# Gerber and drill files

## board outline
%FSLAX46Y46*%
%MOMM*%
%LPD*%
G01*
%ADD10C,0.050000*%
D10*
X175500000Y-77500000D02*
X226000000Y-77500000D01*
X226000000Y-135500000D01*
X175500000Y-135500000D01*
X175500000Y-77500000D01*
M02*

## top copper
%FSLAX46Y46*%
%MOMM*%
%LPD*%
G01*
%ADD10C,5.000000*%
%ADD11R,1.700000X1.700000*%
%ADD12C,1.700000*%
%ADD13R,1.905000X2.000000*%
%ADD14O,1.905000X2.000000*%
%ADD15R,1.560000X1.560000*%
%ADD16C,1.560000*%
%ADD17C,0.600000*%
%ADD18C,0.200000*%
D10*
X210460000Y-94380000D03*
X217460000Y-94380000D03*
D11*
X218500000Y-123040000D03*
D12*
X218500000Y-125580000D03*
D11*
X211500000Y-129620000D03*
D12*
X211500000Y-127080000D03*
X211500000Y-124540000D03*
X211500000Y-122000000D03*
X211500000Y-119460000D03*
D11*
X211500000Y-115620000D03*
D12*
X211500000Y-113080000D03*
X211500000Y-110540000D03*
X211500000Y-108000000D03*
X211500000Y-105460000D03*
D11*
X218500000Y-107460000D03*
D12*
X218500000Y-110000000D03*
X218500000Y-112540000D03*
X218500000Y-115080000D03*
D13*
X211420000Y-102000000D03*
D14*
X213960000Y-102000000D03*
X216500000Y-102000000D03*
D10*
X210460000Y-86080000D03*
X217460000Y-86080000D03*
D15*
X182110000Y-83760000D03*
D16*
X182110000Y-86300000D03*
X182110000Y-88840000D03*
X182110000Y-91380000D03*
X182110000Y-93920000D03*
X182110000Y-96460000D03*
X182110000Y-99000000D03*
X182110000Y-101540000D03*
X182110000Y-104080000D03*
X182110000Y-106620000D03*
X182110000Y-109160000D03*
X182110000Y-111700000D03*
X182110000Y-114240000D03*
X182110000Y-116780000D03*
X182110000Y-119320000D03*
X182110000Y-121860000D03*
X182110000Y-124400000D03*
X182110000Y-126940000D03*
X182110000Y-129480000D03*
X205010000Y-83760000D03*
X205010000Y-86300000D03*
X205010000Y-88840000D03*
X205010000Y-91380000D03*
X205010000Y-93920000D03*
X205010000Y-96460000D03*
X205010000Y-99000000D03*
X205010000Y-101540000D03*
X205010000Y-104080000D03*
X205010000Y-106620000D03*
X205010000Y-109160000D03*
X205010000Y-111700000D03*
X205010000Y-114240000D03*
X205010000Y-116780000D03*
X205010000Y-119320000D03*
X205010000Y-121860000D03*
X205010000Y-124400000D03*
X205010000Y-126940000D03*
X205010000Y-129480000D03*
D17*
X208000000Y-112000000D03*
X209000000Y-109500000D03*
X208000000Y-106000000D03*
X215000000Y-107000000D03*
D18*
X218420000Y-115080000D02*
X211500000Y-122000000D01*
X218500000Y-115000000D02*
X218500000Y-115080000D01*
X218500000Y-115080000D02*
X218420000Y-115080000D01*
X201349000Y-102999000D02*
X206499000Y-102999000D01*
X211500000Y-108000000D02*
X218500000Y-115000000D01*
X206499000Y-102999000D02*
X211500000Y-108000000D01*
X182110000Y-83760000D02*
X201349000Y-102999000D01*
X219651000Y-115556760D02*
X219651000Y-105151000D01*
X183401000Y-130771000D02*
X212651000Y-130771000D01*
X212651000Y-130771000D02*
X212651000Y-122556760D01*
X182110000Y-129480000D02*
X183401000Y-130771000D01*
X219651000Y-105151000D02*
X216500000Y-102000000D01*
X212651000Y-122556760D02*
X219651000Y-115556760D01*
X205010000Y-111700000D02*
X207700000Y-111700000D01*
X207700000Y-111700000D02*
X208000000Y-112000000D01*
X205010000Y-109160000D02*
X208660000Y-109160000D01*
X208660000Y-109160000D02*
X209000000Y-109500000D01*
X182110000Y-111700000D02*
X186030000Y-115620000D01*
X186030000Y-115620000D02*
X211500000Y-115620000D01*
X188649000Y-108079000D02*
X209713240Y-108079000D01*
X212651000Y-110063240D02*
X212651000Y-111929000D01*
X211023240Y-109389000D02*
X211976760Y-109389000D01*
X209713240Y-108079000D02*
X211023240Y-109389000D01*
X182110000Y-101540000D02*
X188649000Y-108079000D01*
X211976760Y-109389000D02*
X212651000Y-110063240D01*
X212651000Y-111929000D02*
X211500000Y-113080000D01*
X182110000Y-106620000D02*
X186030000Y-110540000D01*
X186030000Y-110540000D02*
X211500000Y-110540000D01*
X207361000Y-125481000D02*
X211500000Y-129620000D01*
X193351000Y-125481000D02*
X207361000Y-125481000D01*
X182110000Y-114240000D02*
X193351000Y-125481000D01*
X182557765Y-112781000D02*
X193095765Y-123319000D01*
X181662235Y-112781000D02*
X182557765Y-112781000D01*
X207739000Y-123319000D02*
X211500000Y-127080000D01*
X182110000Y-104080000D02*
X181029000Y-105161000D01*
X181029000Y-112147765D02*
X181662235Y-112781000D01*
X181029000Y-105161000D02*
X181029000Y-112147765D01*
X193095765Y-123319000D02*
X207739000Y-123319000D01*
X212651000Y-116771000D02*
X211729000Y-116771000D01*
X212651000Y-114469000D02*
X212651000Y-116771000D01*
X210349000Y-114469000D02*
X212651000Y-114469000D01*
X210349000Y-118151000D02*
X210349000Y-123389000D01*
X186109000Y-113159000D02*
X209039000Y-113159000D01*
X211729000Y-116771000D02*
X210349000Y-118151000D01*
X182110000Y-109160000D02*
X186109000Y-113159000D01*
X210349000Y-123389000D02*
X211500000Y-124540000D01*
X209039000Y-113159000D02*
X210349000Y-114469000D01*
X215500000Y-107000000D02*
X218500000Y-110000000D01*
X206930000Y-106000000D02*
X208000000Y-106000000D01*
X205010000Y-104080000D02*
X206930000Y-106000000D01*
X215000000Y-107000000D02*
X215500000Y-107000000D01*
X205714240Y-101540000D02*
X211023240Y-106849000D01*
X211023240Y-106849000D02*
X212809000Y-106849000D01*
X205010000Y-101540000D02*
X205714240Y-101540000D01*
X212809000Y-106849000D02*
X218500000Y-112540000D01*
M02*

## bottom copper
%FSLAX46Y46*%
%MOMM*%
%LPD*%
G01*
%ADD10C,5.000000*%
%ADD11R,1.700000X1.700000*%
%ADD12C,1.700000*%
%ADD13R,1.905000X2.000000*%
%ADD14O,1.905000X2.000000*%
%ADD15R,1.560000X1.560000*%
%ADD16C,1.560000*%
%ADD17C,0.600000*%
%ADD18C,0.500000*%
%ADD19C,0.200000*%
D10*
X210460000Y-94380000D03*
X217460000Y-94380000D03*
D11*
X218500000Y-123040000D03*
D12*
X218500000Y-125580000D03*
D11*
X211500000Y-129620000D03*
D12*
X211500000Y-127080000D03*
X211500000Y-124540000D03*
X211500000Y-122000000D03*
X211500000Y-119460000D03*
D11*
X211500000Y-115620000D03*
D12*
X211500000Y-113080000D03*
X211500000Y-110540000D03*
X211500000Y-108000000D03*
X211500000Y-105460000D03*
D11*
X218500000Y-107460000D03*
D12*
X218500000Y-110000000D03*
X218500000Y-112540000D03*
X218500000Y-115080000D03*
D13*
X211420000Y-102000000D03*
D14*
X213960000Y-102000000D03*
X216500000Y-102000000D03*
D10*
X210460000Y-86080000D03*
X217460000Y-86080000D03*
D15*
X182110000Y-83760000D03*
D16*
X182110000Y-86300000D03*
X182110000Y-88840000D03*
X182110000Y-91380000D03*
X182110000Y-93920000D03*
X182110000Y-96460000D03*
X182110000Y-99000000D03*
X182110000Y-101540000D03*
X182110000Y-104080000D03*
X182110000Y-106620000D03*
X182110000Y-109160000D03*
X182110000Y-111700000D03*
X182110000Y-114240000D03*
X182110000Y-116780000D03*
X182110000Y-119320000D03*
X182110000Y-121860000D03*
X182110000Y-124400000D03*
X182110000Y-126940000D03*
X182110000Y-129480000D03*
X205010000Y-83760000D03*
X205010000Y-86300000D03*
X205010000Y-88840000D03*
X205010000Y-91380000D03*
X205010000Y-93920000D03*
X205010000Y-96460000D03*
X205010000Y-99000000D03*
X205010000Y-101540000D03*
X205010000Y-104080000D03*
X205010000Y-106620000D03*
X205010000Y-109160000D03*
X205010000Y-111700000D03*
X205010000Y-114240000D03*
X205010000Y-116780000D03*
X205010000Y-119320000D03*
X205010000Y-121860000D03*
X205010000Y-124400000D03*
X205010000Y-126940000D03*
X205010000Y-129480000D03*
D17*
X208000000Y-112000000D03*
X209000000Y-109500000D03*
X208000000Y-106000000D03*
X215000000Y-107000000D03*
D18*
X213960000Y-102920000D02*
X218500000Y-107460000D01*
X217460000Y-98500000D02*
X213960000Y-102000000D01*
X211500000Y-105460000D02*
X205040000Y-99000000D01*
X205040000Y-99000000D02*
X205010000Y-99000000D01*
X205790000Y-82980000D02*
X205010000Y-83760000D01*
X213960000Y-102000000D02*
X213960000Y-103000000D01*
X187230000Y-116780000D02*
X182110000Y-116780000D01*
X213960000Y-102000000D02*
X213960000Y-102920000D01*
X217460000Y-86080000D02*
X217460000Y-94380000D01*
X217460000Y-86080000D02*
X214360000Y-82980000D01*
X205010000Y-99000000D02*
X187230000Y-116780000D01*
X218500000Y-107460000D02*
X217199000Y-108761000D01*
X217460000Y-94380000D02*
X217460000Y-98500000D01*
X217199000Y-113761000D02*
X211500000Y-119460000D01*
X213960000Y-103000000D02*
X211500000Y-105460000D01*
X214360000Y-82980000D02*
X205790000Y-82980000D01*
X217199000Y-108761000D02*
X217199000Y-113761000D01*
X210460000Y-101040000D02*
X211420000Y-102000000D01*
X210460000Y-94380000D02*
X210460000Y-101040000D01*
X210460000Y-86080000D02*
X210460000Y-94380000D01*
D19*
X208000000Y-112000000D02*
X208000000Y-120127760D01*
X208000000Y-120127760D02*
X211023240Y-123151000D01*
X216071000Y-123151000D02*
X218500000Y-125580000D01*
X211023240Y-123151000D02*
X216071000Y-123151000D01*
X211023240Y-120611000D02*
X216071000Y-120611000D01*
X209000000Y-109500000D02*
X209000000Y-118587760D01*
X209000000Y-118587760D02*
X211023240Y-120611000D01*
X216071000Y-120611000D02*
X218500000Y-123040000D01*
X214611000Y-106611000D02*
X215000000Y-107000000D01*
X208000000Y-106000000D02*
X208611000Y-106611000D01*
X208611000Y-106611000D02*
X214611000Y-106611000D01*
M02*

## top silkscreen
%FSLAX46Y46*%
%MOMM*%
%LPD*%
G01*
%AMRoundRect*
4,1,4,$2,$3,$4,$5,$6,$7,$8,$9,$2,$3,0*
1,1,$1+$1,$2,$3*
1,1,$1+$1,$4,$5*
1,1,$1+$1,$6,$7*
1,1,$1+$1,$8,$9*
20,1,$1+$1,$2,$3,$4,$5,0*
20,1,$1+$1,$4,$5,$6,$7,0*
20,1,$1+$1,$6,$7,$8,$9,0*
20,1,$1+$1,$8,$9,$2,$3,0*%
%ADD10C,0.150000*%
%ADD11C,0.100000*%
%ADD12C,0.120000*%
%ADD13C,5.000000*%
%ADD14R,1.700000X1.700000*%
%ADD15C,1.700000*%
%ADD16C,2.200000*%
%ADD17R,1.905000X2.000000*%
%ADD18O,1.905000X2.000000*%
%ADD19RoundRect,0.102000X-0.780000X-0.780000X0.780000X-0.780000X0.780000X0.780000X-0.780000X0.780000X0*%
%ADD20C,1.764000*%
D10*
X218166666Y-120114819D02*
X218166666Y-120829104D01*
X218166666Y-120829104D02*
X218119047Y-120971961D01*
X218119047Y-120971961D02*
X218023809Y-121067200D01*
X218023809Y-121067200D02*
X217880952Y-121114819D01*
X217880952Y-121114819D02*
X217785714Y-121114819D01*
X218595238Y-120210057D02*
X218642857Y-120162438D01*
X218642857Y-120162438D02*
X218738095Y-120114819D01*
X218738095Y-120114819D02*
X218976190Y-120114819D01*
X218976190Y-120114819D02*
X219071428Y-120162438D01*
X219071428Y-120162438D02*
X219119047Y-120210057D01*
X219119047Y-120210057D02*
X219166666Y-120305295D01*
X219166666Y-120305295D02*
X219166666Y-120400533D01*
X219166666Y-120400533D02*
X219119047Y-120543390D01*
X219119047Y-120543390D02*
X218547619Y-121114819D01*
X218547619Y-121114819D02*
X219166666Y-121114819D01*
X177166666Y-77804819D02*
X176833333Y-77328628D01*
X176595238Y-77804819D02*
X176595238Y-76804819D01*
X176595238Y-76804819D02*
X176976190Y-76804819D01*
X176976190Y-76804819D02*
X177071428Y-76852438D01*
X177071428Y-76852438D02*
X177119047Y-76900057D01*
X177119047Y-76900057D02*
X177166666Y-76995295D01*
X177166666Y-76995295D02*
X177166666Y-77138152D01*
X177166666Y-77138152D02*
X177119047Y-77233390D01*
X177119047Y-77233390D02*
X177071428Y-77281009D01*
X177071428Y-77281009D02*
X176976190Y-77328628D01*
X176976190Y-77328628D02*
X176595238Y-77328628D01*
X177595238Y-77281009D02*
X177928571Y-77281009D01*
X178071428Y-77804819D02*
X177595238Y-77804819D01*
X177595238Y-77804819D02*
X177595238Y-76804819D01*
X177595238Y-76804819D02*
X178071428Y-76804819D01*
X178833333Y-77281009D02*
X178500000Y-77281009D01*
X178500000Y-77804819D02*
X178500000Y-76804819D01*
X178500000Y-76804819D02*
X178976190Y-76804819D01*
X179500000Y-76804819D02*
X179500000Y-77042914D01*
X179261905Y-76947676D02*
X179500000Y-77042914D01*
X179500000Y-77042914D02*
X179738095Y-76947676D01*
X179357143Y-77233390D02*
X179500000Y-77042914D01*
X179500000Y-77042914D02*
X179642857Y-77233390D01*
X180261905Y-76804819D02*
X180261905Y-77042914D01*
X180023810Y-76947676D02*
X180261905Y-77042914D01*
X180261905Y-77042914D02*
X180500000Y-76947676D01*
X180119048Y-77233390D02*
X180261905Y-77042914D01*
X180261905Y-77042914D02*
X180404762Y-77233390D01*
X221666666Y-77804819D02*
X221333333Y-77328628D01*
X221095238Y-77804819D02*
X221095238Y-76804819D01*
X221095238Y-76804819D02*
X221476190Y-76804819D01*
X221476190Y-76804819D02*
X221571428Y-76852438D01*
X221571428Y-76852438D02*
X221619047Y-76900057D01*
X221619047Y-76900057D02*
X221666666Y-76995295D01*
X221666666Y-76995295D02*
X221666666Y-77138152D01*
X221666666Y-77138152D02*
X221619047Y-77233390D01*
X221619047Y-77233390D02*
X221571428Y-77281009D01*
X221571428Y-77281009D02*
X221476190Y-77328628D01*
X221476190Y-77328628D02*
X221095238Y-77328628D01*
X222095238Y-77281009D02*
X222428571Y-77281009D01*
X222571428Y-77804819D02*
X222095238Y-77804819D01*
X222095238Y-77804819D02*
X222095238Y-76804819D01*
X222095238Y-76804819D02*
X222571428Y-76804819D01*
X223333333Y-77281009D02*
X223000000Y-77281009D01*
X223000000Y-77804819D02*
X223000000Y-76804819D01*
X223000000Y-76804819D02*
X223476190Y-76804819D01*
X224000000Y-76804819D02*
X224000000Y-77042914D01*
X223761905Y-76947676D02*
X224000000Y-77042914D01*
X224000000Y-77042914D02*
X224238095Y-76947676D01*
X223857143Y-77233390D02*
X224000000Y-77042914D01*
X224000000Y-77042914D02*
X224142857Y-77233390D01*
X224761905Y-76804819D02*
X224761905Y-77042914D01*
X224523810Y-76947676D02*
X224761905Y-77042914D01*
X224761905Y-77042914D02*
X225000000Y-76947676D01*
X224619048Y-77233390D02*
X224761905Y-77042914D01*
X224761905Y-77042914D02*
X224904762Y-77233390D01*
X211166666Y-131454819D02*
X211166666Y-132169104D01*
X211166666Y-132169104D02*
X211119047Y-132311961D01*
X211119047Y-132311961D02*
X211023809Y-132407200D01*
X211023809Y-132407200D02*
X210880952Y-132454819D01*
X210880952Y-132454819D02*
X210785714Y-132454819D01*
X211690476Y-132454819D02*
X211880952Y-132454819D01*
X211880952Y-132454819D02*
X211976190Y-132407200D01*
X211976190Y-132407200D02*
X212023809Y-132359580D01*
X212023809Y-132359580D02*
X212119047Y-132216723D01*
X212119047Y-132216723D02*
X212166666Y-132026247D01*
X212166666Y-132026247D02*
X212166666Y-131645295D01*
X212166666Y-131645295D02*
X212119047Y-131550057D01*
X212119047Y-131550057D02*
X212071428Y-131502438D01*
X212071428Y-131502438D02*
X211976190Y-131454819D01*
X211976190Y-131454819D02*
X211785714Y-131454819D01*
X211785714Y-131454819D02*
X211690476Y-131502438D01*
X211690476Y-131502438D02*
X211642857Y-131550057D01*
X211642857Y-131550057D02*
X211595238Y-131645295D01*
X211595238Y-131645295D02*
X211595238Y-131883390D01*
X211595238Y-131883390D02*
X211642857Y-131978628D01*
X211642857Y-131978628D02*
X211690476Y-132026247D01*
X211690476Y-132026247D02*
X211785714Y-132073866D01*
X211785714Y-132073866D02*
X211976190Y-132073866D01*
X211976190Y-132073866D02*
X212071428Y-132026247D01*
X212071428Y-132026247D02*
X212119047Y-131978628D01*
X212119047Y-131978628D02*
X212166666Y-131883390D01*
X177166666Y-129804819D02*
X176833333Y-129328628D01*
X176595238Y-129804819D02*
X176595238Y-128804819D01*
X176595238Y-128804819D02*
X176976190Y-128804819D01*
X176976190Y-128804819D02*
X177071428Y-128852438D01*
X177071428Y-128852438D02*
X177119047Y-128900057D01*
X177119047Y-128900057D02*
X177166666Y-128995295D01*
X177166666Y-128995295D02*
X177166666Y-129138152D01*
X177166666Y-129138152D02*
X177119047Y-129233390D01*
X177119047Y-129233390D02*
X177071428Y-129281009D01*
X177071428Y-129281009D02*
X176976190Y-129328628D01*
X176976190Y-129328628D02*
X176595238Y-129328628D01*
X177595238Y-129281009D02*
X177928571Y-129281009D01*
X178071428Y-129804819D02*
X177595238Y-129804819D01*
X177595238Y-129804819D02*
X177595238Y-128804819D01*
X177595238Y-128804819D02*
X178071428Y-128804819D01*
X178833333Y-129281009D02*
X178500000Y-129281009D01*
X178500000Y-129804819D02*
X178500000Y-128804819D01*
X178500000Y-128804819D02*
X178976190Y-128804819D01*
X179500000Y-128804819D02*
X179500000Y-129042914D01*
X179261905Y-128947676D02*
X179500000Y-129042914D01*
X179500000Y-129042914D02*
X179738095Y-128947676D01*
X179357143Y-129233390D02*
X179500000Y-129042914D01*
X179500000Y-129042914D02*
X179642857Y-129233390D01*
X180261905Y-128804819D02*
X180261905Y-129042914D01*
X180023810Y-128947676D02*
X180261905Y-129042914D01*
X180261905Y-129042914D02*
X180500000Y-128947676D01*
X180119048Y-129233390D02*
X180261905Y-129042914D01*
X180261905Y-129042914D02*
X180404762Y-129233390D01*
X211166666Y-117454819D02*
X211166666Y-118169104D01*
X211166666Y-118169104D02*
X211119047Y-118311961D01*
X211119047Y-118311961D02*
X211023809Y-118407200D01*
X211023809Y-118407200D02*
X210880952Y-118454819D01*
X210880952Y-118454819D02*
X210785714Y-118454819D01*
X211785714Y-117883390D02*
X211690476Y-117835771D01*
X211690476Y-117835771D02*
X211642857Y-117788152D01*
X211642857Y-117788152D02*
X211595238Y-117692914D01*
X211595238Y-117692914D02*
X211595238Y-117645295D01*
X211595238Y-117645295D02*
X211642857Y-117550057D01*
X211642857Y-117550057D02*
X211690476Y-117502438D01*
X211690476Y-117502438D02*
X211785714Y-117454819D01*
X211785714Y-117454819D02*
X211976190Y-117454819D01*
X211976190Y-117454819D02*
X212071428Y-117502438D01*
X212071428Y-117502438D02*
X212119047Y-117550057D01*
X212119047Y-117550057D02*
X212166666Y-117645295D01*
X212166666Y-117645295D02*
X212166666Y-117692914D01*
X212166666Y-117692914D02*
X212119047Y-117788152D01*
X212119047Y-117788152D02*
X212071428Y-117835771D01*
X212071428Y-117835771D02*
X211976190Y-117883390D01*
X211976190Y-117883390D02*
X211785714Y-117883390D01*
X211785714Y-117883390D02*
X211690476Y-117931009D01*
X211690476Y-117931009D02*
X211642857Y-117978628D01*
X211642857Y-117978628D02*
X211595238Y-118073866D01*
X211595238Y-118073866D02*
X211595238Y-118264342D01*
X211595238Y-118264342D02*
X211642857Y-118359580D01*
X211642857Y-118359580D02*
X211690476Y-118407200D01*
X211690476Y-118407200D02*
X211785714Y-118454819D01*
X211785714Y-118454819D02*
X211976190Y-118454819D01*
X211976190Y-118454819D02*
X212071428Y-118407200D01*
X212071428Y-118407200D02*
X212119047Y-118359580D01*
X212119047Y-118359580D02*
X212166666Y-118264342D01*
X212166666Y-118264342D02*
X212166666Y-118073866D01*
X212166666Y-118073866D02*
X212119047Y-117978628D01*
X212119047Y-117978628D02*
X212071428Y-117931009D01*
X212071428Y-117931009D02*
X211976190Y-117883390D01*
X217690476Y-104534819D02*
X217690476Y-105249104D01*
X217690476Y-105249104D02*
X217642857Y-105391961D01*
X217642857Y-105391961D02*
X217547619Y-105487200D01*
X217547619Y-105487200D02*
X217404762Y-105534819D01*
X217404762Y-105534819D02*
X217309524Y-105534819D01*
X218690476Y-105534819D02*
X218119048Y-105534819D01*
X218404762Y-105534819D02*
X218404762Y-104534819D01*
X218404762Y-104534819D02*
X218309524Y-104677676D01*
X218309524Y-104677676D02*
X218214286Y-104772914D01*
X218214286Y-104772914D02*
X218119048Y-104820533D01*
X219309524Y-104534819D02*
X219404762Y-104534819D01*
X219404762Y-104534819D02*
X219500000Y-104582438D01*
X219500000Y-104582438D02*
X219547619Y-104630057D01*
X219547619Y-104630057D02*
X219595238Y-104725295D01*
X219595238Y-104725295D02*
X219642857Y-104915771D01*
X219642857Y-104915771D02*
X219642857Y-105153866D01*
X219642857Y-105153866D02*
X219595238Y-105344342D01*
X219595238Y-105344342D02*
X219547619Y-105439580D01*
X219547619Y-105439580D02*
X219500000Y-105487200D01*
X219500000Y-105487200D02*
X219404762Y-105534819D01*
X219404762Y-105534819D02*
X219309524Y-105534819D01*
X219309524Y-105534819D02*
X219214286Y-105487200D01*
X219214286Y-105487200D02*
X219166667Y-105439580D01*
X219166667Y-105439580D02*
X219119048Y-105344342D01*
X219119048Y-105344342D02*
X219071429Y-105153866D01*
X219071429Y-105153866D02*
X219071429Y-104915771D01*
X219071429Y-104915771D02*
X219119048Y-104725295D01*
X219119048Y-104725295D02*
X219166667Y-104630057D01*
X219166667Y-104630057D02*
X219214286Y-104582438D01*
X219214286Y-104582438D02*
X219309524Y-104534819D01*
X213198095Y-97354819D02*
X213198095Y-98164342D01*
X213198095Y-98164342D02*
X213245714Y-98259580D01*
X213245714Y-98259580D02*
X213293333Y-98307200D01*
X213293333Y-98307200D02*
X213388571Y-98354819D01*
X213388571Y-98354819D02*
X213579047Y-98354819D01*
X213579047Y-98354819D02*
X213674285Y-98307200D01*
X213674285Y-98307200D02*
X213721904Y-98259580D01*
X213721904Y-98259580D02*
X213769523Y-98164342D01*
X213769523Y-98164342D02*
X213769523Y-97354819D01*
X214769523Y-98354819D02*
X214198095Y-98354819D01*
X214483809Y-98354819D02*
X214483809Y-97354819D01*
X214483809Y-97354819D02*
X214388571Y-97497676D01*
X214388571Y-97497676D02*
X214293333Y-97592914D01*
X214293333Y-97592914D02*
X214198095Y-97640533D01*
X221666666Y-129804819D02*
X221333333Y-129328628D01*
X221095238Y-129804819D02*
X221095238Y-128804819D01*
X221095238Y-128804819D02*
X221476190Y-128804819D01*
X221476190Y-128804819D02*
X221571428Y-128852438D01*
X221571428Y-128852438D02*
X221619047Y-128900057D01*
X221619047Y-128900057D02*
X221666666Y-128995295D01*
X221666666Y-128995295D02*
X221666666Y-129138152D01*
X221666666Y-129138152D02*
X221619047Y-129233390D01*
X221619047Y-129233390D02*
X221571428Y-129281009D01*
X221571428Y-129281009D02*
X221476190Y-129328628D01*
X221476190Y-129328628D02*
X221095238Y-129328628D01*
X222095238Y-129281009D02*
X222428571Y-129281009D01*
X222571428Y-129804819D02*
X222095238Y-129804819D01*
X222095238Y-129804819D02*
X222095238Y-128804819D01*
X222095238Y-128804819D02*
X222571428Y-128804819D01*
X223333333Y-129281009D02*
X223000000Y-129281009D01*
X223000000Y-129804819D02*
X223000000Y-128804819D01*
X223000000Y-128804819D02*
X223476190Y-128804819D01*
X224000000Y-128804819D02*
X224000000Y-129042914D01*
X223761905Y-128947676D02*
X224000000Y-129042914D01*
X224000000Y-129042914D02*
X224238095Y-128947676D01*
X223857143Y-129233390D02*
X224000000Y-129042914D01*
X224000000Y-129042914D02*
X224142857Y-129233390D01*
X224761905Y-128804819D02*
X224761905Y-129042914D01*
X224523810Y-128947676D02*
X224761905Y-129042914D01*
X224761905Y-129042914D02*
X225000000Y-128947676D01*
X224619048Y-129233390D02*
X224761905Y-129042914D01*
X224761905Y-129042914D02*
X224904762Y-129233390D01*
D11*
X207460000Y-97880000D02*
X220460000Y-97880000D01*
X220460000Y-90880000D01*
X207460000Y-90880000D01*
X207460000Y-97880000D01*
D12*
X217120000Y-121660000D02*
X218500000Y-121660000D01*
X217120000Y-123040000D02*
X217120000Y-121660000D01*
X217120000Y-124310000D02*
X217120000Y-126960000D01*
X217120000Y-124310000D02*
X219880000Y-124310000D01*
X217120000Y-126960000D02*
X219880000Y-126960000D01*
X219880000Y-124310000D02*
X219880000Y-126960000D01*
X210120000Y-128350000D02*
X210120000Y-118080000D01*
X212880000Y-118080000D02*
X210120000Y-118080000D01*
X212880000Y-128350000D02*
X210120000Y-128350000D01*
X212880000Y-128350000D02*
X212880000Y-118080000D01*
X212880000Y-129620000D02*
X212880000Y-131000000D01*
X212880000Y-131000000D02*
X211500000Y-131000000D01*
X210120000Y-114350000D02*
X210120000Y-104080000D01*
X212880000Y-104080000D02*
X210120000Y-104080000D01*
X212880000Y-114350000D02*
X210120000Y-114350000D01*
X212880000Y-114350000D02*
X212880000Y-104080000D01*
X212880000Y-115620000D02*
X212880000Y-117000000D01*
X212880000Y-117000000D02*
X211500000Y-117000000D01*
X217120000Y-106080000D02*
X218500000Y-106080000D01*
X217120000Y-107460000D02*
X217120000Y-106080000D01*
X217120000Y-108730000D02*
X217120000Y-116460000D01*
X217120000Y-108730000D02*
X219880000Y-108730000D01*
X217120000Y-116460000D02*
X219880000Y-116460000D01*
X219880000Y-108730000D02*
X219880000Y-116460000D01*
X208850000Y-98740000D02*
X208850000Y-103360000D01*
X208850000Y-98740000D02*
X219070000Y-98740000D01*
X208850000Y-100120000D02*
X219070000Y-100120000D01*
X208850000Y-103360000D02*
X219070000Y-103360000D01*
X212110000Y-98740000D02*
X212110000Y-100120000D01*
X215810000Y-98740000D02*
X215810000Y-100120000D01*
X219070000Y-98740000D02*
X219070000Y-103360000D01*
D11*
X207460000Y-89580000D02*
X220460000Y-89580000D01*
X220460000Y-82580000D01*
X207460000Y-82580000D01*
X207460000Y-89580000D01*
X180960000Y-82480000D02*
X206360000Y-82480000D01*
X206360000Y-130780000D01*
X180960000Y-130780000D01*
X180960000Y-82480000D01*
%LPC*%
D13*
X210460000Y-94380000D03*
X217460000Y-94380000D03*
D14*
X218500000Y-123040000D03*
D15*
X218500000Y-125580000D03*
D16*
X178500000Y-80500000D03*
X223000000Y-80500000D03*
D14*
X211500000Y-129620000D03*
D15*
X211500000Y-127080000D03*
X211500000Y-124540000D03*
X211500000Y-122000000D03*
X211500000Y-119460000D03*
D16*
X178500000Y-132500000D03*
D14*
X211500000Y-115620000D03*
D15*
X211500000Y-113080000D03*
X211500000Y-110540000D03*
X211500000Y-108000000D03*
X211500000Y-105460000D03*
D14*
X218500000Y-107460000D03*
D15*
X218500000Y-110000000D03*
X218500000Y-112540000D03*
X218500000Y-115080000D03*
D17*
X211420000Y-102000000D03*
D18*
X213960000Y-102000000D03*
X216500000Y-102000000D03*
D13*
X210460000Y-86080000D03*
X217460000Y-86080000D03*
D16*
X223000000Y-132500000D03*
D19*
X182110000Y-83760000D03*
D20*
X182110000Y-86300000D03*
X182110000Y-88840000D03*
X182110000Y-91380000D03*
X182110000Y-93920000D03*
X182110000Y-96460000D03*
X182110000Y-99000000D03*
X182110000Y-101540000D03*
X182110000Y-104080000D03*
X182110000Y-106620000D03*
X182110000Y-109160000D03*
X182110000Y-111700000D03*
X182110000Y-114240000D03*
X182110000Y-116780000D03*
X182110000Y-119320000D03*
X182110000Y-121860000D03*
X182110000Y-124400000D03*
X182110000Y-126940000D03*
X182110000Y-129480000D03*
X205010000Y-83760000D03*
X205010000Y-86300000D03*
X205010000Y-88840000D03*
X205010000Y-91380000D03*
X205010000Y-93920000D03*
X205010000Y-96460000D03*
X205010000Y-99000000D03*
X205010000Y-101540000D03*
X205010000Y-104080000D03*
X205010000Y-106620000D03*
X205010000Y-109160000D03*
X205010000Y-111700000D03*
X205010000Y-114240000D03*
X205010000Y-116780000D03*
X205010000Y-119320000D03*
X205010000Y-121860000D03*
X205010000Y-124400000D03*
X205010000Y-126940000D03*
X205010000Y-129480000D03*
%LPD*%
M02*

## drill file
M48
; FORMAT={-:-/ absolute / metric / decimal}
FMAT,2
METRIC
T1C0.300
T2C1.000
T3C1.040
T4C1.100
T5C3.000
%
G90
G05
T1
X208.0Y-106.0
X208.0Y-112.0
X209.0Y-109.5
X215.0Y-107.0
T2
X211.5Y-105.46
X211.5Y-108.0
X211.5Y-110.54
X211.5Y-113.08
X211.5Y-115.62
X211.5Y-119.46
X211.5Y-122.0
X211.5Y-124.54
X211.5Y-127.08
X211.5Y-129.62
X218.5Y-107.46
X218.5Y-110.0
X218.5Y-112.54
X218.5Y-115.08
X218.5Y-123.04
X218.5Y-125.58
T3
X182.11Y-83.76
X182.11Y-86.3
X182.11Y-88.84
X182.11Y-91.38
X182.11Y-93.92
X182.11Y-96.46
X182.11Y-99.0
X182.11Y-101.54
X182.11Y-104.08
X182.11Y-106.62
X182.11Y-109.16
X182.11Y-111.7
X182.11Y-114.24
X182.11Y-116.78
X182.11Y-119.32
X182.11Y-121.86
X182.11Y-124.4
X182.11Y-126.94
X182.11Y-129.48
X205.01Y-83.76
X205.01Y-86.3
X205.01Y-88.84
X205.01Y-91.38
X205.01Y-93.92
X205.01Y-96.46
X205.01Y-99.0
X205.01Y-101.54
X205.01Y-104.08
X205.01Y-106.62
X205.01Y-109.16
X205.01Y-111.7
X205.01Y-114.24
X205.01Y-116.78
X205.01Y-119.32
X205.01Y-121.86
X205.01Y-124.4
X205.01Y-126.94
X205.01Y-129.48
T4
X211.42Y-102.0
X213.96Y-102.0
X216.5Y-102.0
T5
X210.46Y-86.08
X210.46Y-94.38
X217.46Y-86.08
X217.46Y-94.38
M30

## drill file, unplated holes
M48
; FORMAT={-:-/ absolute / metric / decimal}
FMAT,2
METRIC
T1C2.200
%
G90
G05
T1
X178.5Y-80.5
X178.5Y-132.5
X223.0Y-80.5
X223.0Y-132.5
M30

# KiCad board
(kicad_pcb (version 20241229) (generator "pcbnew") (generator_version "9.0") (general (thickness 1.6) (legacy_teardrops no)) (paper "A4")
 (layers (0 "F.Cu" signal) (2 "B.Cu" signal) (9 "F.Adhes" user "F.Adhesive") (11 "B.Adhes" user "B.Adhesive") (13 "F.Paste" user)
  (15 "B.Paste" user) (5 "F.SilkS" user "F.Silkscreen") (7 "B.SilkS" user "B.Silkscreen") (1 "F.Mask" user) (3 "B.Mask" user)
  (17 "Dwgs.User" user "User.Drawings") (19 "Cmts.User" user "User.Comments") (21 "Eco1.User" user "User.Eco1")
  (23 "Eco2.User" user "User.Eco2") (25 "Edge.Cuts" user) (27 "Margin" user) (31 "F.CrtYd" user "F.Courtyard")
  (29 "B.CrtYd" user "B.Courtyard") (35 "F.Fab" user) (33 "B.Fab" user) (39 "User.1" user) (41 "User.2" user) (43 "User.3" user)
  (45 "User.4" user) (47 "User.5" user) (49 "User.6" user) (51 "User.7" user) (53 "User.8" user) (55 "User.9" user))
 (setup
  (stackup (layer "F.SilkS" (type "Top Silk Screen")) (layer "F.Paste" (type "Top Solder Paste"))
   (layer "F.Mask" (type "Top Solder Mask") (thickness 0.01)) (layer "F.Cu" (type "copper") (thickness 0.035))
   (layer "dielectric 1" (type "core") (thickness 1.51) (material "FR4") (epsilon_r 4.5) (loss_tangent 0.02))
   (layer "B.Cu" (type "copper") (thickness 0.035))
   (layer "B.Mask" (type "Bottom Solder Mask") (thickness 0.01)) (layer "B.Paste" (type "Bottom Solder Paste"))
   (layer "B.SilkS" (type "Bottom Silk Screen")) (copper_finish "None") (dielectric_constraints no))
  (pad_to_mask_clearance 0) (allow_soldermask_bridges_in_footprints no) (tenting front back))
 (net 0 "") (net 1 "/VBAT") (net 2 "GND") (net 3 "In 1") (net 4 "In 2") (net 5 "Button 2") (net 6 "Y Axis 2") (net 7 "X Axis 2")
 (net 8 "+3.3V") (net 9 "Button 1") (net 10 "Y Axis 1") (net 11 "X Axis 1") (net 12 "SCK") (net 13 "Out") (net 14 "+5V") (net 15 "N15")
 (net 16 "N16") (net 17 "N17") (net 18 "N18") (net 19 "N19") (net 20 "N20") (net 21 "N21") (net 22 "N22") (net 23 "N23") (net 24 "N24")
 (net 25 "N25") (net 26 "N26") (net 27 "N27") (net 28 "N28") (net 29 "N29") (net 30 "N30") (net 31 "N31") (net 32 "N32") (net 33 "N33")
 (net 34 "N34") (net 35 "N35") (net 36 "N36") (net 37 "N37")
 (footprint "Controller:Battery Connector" (layer "F.Cu") (at 220.96 94.38 90)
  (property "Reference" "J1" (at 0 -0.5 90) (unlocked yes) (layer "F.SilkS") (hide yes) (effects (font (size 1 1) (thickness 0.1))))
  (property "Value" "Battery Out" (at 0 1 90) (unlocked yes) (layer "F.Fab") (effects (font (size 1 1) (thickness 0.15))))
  (fp_rect (start -3.5 -13.5) (end 3.5 -0.5) (stroke (width 0.1) (type default)) (fill no) (layer "F.SilkS"))
  (pad "1" thru_hole circle (at 0 -10.5 90) (size 5 5) (drill 3) (layers "*.Cu" "*.Mask") (remove_unused_layers no) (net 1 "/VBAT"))
  (pad "2" thru_hole circle (at 0 -3.5 90) (size 5 5) (drill 3) (layers "*.Cu" "*.Mask") (remove_unused_layers no) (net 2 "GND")))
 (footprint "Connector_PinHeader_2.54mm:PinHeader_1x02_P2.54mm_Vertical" (layer "F.Cu") (at 218.5 123.04)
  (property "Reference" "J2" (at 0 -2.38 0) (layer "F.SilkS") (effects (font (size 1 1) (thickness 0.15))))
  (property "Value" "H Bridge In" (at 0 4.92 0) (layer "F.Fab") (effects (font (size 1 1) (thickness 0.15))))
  (fp_line (start -1.38 -1.38) (end 0 -1.38) (stroke (width 0.12) (type solid)) (layer "F.SilkS"))
  (fp_line (start -1.38 0) (end -1.38 -1.38) (stroke (width 0.12) (type solid)) (layer "F.SilkS"))
  (fp_line (start -1.38 1.27) (end -1.38 3.92) (stroke (width 0.12) (type solid)) (layer "F.SilkS"))
  (fp_line (start -1.38 1.27) (end 1.38 1.27) (stroke (width 0.12) (type solid)) (layer "F.SilkS"))
  (fp_line (start -1.38 3.92) (end 1.38 3.92) (stroke (width 0.12) (type solid)) (layer "F.SilkS"))
  (fp_line (start 1.38 1.27) (end 1.38 3.92) (stroke (width 0.12) (type solid)) (layer "F.SilkS"))
  (pad "1" thru_hole rect (at 0 0) (size 1.7 1.7) (drill 1) (layers "*.Cu" "*.Mask") (remove_unused_layers no) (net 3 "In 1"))
  (pad "2" thru_hole circle (at 0 2.54) (size 1.7 1.7) (drill 1) (layers "*.Cu" "*.Mask") (remove_unused_layers no) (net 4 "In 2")))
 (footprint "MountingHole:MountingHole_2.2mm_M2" (layer "F.Cu") (at 178.5 80.5)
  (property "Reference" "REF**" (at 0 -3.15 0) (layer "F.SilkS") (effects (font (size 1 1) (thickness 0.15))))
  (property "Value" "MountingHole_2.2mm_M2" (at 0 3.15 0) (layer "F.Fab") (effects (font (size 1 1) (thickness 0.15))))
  (pad "" np_thru_hole circle (at 0 0) (size 2.2 2.2) (drill 2.2) (layers "*.Cu" "*.Mask")))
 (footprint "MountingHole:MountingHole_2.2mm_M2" (layer "F.Cu") (at 223 80.5)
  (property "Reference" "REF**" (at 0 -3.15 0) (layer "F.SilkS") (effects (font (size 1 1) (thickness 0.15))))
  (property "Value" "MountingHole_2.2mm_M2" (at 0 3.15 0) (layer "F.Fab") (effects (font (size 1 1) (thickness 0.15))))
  (pad "" np_thru_hole circle (at 0 0) (size 2.2 2.2) (drill 2.2) (layers "*.Cu" "*.Mask")))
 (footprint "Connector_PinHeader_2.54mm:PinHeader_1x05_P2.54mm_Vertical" (layer "F.Cu") (at 211.5 129.62 180)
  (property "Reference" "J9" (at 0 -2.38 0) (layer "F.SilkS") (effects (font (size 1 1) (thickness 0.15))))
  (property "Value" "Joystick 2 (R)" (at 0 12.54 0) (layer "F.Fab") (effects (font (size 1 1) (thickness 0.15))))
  (fp_line (start 1.38 1.27) (end 1.38 11.54) (stroke (width 0.12) (type solid)) (layer "F.SilkS"))
  (fp_line (start -1.38 11.54) (end 1.38 11.54) (stroke (width 0.12) (type solid)) (layer "F.SilkS"))
  (fp_line (start -1.38 1.27) (end 1.38 1.27) (stroke (width 0.12) (type solid)) (layer "F.SilkS"))
  (fp_line (start -1.38 1.27) (end -1.38 11.54) (stroke (width 0.12) (type solid)) (layer "F.SilkS"))
  (fp_line (start -1.38 0) (end -1.38 -1.38) (stroke (width 0.12) (type solid)) (layer "F.SilkS"))
  (fp_line (start -1.38 -1.38) (end 0 -1.38) (stroke (width 0.12) (type solid)) (layer "F.SilkS"))
  (pad "1" thru_hole rect (at 0 0 180) (size 1.7 1.7) (drill 1) (layers "*.Cu" "*.Mask") (remove_unused_layers no) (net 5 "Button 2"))
  (pad "2" thru_hole circle (at 0 2.54 180) (size 1.7 1.7) (drill 1) (layers "*.Cu" "*.Mask") (remove_unused_layers no) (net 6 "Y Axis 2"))
  (pad "3" thru_hole circle (at 0 5.08 180) (size 1.7 1.7) (drill 1) (layers "*.Cu" "*.Mask") (remove_unused_layers no) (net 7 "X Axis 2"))
  (pad "4" thru_hole circle (at 0 7.62 180) (size 1.7 1.7) (drill 1) (layers "*.Cu" "*.Mask") (remove_unused_layers no) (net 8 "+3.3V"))
  (pad "5" thru_hole circle (at 0 10.16 180) (size 1.7 1.7) (drill 1) (layers "*.Cu" "*.Mask") (remove_unused_layers no) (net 2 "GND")))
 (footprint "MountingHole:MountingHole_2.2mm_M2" (layer "F.Cu") (at 178.5 132.5)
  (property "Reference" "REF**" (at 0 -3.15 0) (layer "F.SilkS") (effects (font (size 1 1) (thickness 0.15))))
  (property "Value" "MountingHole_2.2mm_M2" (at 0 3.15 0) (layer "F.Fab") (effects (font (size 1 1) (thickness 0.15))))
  (pad "" np_thru_hole circle (at 0 0) (size 2.2 2.2) (drill 2.2) (layers "*.Cu" "*.Mask")))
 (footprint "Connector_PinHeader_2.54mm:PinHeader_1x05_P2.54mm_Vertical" (layer "F.Cu") (at 211.5 115.62 180)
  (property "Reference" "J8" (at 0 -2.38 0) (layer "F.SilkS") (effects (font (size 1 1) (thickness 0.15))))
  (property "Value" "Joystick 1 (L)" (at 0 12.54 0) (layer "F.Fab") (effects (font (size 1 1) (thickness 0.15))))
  (fp_line (start 1.38 1.27) (end 1.38 11.54) (stroke (width 0.12) (type solid)) (layer "F.SilkS"))
  (fp_line (start -1.38 11.54) (end 1.38 11.54) (stroke (width 0.12) (type solid)) (layer "F.SilkS"))
  (fp_line (start -1.38 1.27) (end 1.38 1.27) (stroke (width 0.12) (type solid)) (layer "F.SilkS"))
  (fp_line (start -1.38 1.27) (end -1.38 11.54) (stroke (width 0.12) (type solid)) (layer "F.SilkS"))
  (fp_line (start -1.38 0) (end -1.38 -1.38) (stroke (width 0.12) (type solid)) (layer "F.SilkS"))
  (fp_line (start -1.38 -1.38) (end 0 -1.38) (stroke (width 0.12) (type solid)) (layer "F.SilkS"))
  (pad "1" thru_hole rect (at 0 0 180) (size 1.7 1.7) (drill 1) (layers "*.Cu" "*.Mask") (remove_unused_layers no) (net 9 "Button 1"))
  (pad "2" thru_hole circle (at 0 2.54 180) (size 1.7 1.7) (drill 1) (layers "*.Cu" "*.Mask") (remove_unused_layers no) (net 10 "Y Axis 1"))
  (pad "3" thru_hole circle (at 0 5.08 180) (size 1.7 1.7) (drill 1) (layers "*.Cu" "*.Mask") (remove_unused_layers no) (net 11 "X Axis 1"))
  (pad "4" thru_hole circle (at 0 7.62 180) (size 1.7 1.7) (drill 1) (layers "*.Cu" "*.Mask") (remove_unused_layers no) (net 8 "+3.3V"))
  (pad "5" thru_hole circle (at 0 10.16 180) (size 1.7 1.7) (drill 1) (layers "*.Cu" "*.Mask") (remove_unused_layers no) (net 2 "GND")))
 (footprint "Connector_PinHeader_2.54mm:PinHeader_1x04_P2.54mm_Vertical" (layer "F.Cu") (at 218.5 107.46)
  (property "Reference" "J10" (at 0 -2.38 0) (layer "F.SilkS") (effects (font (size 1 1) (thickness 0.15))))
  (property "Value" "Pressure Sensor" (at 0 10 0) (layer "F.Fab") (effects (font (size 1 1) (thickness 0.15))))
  (fp_line (start -1.38 -1.38) (end 0 -1.38) (stroke (width 0.12) (type solid)) (layer "F.SilkS"))
  (fp_line (start -1.38 0) (end -1.38 -1.38) (stroke (width 0.12) (type solid)) (layer "F.SilkS"))
  (fp_line (start -1.38 1.27) (end -1.38 9) (stroke (width 0.12) (type solid)) (layer "F.SilkS"))
  (fp_line (start -1.38 1.27) (end 1.38 1.27) (stroke (width 0.12) (type solid)) (layer "F.SilkS"))
  (fp_line (start -1.38 9) (end 1.38 9) (stroke (width 0.12) (type solid)) (layer "F.SilkS"))
  (fp_line (start 1.38 1.27) (end 1.38 9) (stroke (width 0.12) (type solid)) (layer "F.SilkS"))
  (pad "1" thru_hole rect (at 0 0) (size 1.7 1.7) (drill 1) (layers "*.Cu" "*.Mask") (remove_unused_layers no) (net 2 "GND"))
  (pad "2" thru_hole circle (at 0 2.54) (size 1.7 1.7) (drill 1) (layers "*.Cu" "*.Mask") (remove_unused_layers no) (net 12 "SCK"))
  (pad "3" thru_hole circle (at 0 5.08) (size 1.7 1.7) (drill 1) (layers "*.Cu" "*.Mask") (remove_unused_layers no) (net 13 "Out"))
  (pad "4" thru_hole circle (at 0 7.62) (size 1.7 1.7) (drill 1) (layers "*.Cu" "*.Mask") (remove_unused_layers no) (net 8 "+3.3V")))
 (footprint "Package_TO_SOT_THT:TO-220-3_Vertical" (layer "F.Cu") (at 211.42 102)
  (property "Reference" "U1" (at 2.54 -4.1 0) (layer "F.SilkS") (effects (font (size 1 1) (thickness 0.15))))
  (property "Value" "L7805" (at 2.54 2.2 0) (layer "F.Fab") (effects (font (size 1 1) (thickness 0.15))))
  (fp_line (start -2.57 -3.26) (end -2.57 1.36) (stroke (width 0.12) (type solid)) (layer "F.SilkS"))
  (fp_line (start -2.57 -3.26) (end 7.65 -3.26) (stroke (width 0.12) (type solid)) (layer "F.SilkS"))
  (fp_line (start -2.57 -1.88) (end 7.65 -1.88) (stroke (width 0.12) (type solid)) (layer "F.SilkS"))
  (fp_line (start -2.57 1.36) (end 7.65 1.36) (stroke (width 0.12) (type solid)) (layer "F.SilkS"))
  (fp_line (start 0.69 -3.26) (end 0.69 -1.88) (stroke (width 0.12) (type solid)) (layer "F.SilkS"))
  (fp_line (start 4.39 -3.26) (end 4.39 -1.88) (stroke (width 0.12) (type solid)) (layer "F.SilkS"))
  (fp_line (start 7.65 -3.26) (end 7.65 1.36) (stroke (width 0.12) (type solid)) (layer "F.SilkS"))
  (pad "1" thru_hole rect (at 0 0) (size 1.905 2) (drill 1.1) (layers "*.Cu" "*.Mask") (remove_unused_layers no) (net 1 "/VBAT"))
  (pad "2" thru_hole oval (at 2.54 0) (size 1.905 2) (drill 1.1) (layers "*.Cu" "*.Mask") (remove_unused_layers no) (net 2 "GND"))
  (pad "3" thru_hole oval (at 5.08 0) (size 1.905 2) (drill 1.1) (layers "*.Cu" "*.Mask") (remove_unused_layers no) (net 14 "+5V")))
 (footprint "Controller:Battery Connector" (layer "F.Cu") (at 220.96 86.08 90)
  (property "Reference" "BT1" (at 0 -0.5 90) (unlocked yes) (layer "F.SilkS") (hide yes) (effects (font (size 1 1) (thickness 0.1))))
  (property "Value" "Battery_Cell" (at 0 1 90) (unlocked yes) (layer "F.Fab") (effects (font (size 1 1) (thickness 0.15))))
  (fp_rect (start -3.5 -13.5) (end 3.5 -0.5) (stroke (width 0.1) (type default)) (fill no) (layer "F.SilkS"))
  (pad "1" thru_hole circle (at 0 -10.5 90) (size 5 5) (drill 3) (layers "*.Cu" "*.Mask") (remove_unused_layers no) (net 1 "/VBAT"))
  (pad "2" thru_hole circle (at 0 -3.5 90) (size 5 5) (drill 3) (layers "*.Cu" "*.Mask") (remove_unused_layers no) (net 2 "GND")))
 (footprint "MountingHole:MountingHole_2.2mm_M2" (layer "F.Cu") (at 223 132.5)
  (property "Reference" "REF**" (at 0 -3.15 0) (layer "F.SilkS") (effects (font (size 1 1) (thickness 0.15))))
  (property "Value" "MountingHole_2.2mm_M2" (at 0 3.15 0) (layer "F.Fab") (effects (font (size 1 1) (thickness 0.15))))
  (pad "" np_thru_hole circle (at 0 0) (size 2.2 2.2) (drill 2.2) (layers "*.Cu" "*.Mask")))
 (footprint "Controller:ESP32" (layer "F.Cu") (at 193.36 107.28)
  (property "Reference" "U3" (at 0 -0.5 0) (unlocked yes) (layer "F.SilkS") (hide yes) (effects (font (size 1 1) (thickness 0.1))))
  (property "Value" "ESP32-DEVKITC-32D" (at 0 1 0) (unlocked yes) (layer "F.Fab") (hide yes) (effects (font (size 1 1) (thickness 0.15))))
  (fp_rect (start -12.4 -24.8) (end 13 23.5) (stroke (width 0.1) (type default)) (fill no) (layer "F.SilkS"))
  (pad "J2-1" thru_hole rect (at -11.25 -23.52) (size 1.56 1.56) (drill 1.04) (layers "*.Cu" "*.Mask") (remove_unused_layers no)
   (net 8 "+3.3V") (solder_mask_margin 0.102))
  (pad "J2-2" thru_hole circle (at -11.25 -20.98) (size 1.56 1.56) (drill 1.04) (layers "*.Cu" "*.Mask") (remove_unused_layers no)
   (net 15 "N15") (solder_mask_margin 0.102))
  (pad "J2-3" thru_hole circle (at -11.25 -18.44) (size 1.56 1.56) (drill 1.04) (layers "*.Cu" "*.Mask") (remove_unused_layers no)
   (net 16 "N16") (solder_mask_margin 0.102))
  (pad "J2-4" thru_hole circle (at -11.25 -15.9) (size 1.56 1.56) (drill 1.04) (layers "*.Cu" "*.Mask") (remove_unused_layers no)
   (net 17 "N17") (solder_mask_margin 0.102))
  (pad "J2-5" thru_hole circle (at -11.25 -13.36) (size 1.56 1.56) (drill 1.04) (layers "*.Cu" "*.Mask") (remove_unused_layers no)
   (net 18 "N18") (solder_mask_margin 0.102))
  (pad "J2-6" thru_hole circle (at -11.25 -10.82) (size 1.56 1.56) (drill 1.04) (layers "*.Cu" "*.Mask") (remove_unused_layers no)
   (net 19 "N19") (solder_mask_margin 0.102))
  (pad "J2-7" thru_hole circle (at -11.25 -8.28) (size 1.56 1.56) (drill 1.04) (layers "*.Cu" "*.Mask") (remove_unused_layers no)
   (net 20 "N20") (solder_mask_margin 0.102))
  (pad "J2-8" thru_hole circle (at -11.25 -5.74) (size 1.56 1.56) (drill 1.04) (layers "*.Cu" "*.Mask") (remove_unused_layers no)
   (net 10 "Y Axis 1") (solder_mask_margin 0.102))
  (pad "J2-9" thru_hole circle (at -11.25 -3.2) (size 1.56 1.56) (drill 1.04) (layers "*.Cu" "*.Mask") (remove_unused_layers no)
   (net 6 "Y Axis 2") (solder_mask_margin 0.102))
  (pad "J2-10" thru_hole circle (at -11.25 -0.66) (size 1.56 1.56) (drill 1.04) (layers "*.Cu" "*.Mask") (remove_unused_layers no)
   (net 11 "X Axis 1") (solder_mask_margin 0.102))
  (pad "J2-11" thru_hole circle (at -11.25 1.88) (size 1.56 1.56) (drill 1.04) (layers "*.Cu" "*.Mask") (remove_unused_layers no)
   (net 7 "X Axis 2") (solder_mask_margin 0.102))
  (pad "J2-12" thru_hole circle (at -11.25 4.42) (size 1.56 1.56) (drill 1.04) (layers "*.Cu" "*.Mask") (remove_unused_layers no)
   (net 9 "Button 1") (solder_mask_margin 0.102))
  (pad "J2-13" thru_hole circle (at -11.25 6.96) (size 1.56 1.56) (drill 1.04) (layers "*.Cu" "*.Mask") (remove_unused_layers no)
   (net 5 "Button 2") (solder_mask_margin 0.102))
  (pad "J2-14" thru_hole circle (at -11.25 9.5) (size 1.56 1.56) (drill 1.04) (layers "*.Cu" "*.Mask") (remove_unused_layers no)
   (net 2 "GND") (solder_mask_margin 0.102))
  (pad "J2-15" thru_hole circle (at -11.25 12.04) (size 1.56 1.56) (drill 1.04) (layers "*.Cu" "*.Mask") (remove_unused_layers no)
   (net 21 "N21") (solder_mask_margin 0.102))
  (pad "J2-16" thru_hole circle (at -11.25 14.58) (size 1.56 1.56) (drill 1.04) (layers "*.Cu" "*.Mask") (remove_unused_layers no)
   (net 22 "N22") (solder_mask_margin 0.102))
  (pad "J2-17" thru_hole circle (at -11.25 17.12) (size 1.56 1.56) (drill 1.04) (layers "*.Cu" "*.Mask") (remove_unused_layers no)
   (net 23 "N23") (solder_mask_margin 0.102))
  (pad "J2-18" thru_hole circle (at -11.25 19.66) (size 1.56 1.56) (drill 1.04) (layers "*.Cu" "*.Mask") (remove_unused_layers no)
   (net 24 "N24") (solder_mask_margin 0.102))
  (pad "J2-19" thru_hole circle (at -11.25 22.2) (size 1.56 1.56) (drill 1.04) (layers "*.Cu" "*.Mask") (remove_unused_layers no)
   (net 14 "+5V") (solder_mask_margin 0.102))
  (pad "J3-1" thru_hole circle (at 11.65 -23.52) (size 1.56 1.56) (drill 1.04) (layers "*.Cu" "*.Mask") (remove_unused_layers no)
   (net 2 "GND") (solder_mask_margin 0.102))
  (pad "J3-2" thru_hole circle (at 11.65 -20.98) (size 1.56 1.56) (drill 1.04) (layers "*.Cu" "*.Mask") (remove_unused_layers no)
   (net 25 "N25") (solder_mask_margin 0.102))
  (pad "J3-3" thru_hole circle (at 11.65 -18.44) (size 1.56 1.56) (drill 1.04) (layers "*.Cu" "*.Mask") (remove_unused_layers no)
   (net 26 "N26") (solder_mask_margin 0.102))
  (pad "J3-4" thru_hole circle (at 11.65 -15.9) (size 1.56 1.56) (drill 1.04) (layers "*.Cu" "*.Mask") (remove_unused_layers no)
   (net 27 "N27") (solder_mask_margin 0.102))
  (pad "J3-5" thru_hole circle (at 11.65 -13.36) (size 1.56 1.56) (drill 1.04) (layers "*.Cu" "*.Mask") (remove_unused_layers no)
   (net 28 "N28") (solder_mask_margin 0.102))
  (pad "J3-6" thru_hole circle (at 11.65 -10.82) (size 1.56 1.56) (drill 1.04) (layers "*.Cu" "*.Mask") (remove_unused_layers no)
   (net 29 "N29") (solder_mask_margin 0.102))
  (pad "J3-7" thru_hole circle (at 11.65 -8.28) (size 1.56 1.56) (drill 1.04) (layers "*.Cu" "*.Mask") (remove_unused_layers no)
   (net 2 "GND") (solder_mask_margin 0.102))
  (pad "J3-8" thru_hole circle (at 11.65 -5.74) (size 1.56 1.56) (drill 1.04) (layers "*.Cu" "*.Mask") (remove_unused_layers no)
   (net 13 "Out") (solder_mask_margin 0.102))
  (pad "J3-9" thru_hole circle (at 11.65 -3.2) (size 1.56 1.56) (drill 1.04) (layers "*.Cu" "*.Mask") (remove_unused_layers no)
   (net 12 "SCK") (solder_mask_margin 0.102))
  (pad "J3-10" thru_hole circle (at 11.65 -0.66) (size 1.56 1.56) (drill 1.04) (layers "*.Cu" "*.Mask") (remove_unused_layers no)
   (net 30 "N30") (solder_mask_margin 0.102))
  (pad "J3-11" thru_hole circle (at 11.65 1.88) (size 1.56 1.56) (drill 1.04) (layers "*.Cu" "*.Mask") (remove_unused_layers no)
   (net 3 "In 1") (solder_mask_margin 0.102))
  (pad "J3-12" thru_hole circle (at 11.65 4.42) (size 1.56 1.56) (drill 1.04) (layers "*.Cu" "*.Mask") (remove_unused_layers no)
   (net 4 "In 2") (solder_mask_margin 0.102))
  (pad "J3-13" thru_hole circle (at 11.65 6.96) (size 1.56 1.56) (drill 1.04) (layers "*.Cu" "*.Mask") (remove_unused_layers no)
   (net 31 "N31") (solder_mask_margin 0.102))
  (pad "J3-14" thru_hole circle (at 11.65 9.5) (size 1.56 1.56) (drill 1.04) (layers "*.Cu" "*.Mask") (remove_unused_layers no)
   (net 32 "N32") (solder_mask_margin 0.102))
  (pad "J3-15" thru_hole circle (at 11.65 12.04) (size 1.56 1.56) (drill 1.04) (layers "*.Cu" "*.Mask") (remove_unused_layers no)
   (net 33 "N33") (solder_mask_margin 0.102))
  (pad "J3-16" thru_hole circle (at 11.65 14.58) (size 1.56 1.56) (drill 1.04) (layers "*.Cu" "*.Mask") (remove_unused_layers no)
   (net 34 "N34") (solder_mask_margin 0.102))
  (pad "J3-17" thru_hole circle (at 11.65 17.12) (size 1.56 1.56) (drill 1.04) (layers "*.Cu" "*.Mask") (remove_unused_layers no)
   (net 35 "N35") (solder_mask_margin 0.102))
  (pad "J3-18" thru_hole circle (at 11.65 19.66) (size 1.56 1.56) (drill 1.04) (layers "*.Cu" "*.Mask") (remove_unused_layers no)
   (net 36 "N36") (solder_mask_margin 0.102))
  (pad "J3-19" thru_hole circle (at 11.65 22.2) (size 1.56 1.56) (drill 1.04) (layers "*.Cu" "*.Mask") (remove_unused_layers no)
   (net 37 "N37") (solder_mask_margin 0.102)))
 (gr_rect (start 175.5 77.5) (end 226 135.5) (stroke (width 0.05) (type default)) (fill no) (layer "Edge.Cuts"))
 (segment (start 213.96 102.92) (end 218.5 107.46) (width 0.5) (layer "B.Cu") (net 2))
 (segment (start 217.46 98.5) (end 213.96 102) (width 0.5) (layer "B.Cu") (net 2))
 (segment (start 211.5 105.46) (end 205.04 99) (width 0.5) (layer "B.Cu") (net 2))
 (segment (start 205.04 99) (end 205.01 99) (width 0.5) (layer "B.Cu") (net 2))
 (segment (start 205.79 82.98) (end 205.01 83.76) (width 0.5) (layer "B.Cu") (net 2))
 (segment (start 213.96 102) (end 213.96 103) (width 0.5) (layer "B.Cu") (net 2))
 (segment (start 187.23 116.78) (end 182.11 116.78) (width 0.5) (layer "B.Cu") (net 2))
 (segment (start 213.96 102) (end 213.96 102.92) (width 0.5) (layer "B.Cu") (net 2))
 (segment (start 217.46 86.08) (end 217.46 94.38) (width 0.5) (layer "B.Cu") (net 2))
 (segment (start 217.46 86.08) (end 214.36 82.98) (width 0.5) (layer "B.Cu") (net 2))
 (segment (start 205.01 99) (end 187.23 116.78) (width 0.5) (layer "B.Cu") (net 2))
 (segment (start 218.5 107.46) (end 217.199 108.761) (width 0.5) (layer "B.Cu") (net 2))
 (segment (start 217.46 94.38) (end 217.46 98.5) (width 0.5) (layer "B.Cu") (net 2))
 (segment (start 217.199 113.761) (end 211.5 119.46) (width 0.5) (layer "B.Cu") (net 2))
 (segment (start 213.96 103) (end 211.5 105.46) (width 0.5) (layer "B.Cu") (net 2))
 (segment (start 214.36 82.98) (end 205.79 82.98) (width 0.5) (layer "B.Cu") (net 2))
 (segment (start 217.199 108.761) (end 217.199 113.761) (width 0.5) (layer "B.Cu") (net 2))
 (segment (start 210.46 101.04) (end 211.42 102) (width 0.5) (layer "B.Cu") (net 1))
 (segment (start 210.46 94.38) (end 210.46 101.04) (width 0.5) (layer "B.Cu") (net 1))
 (segment (start 210.46 86.08) (end 210.46 94.38) (width 0.5) (layer "B.Cu") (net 1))
 (segment (start 218.42 115.08) (end 211.5 122) (width 0.2) (layer "F.Cu") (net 8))
 (segment (start 218.5 115) (end 218.5 115.08) (width 0.2) (layer "F.Cu") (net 8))
 (segment (start 218.5 115.08) (end 218.42 115.08) (width 0.2) (layer "F.Cu") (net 8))
 (segment (start 201.349 102.999) (end 206.499 102.999) (width 0.2) (layer "F.Cu") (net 8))
 (segment (start 211.5 108) (end 218.5 115) (width 0.2) (layer "F.Cu") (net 8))
 (segment (start 206.499 102.999) (end 211.5 108) (width 0.2) (layer "F.Cu") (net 8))
 (segment (start 182.11 83.76) (end 201.349 102.999) (width 0.2) (layer "F.Cu") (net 8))
 (segment (start 219.651 115.55676) (end 219.651 105.151) (width 0.2) (layer "F.Cu") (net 14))
 (segment (start 183.401 130.771) (end 212.651 130.771) (width 0.2) (layer "F.Cu") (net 14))
 (segment (start 212.651 130.771) (end 212.651 122.55676) (width 0.2) (layer "F.Cu") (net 14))
 (segment (start 182.11 129.48) (end 183.401 130.771) (width 0.2) (layer "F.Cu") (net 14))
 (segment (start 219.651 105.151) (end 216.5 102) (width 0.2) (layer "F.Cu") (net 14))
 (segment (start 212.651 122.55676) (end 219.651 115.55676) (width 0.2) (layer "F.Cu") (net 14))
 (segment (start 205.01 111.7) (end 207.7 111.7) (width 0.2) (layer "F.Cu") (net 4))
 (segment (start 207.7 111.7) (end 208 112) (width 0.2) (layer "F.Cu") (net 4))
 (via (at 208 112) (size 0.6) (drill 0.3) (layers "F.Cu" "B.Cu") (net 4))
 (segment (start 208 112) (end 208 120.12776) (width 0.2) (layer "B.Cu") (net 4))
 (segment (start 208 120.12776) (end 211.02324 123.151) (width 0.2) (layer "B.Cu") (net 4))
 (segment (start 216.071 123.151) (end 218.5 125.58) (width 0.2) (layer "B.Cu") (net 4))
 (segment (start 211.02324 123.151) (end 216.071 123.151) (width 0.2) (layer "B.Cu") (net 4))
 (segment (start 205.01 109.16) (end 208.66 109.16) (width 0.2) (layer "F.Cu") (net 3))
 (segment (start 208.66 109.16) (end 209 109.5) (width 0.2) (layer "F.Cu") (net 3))
 (via (at 209 109.5) (size 0.6) (drill 0.3) (layers "F.Cu" "B.Cu") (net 3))
 (segment (start 211.02324 120.611) (end 216.071 120.611) (width 0.2) (layer "B.Cu") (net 3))
 (segment (start 209 109.5) (end 209 118.58776) (width 0.2) (layer "B.Cu") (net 3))
 (segment (start 209 118.58776) (end 211.02324 120.611) (width 0.2) (layer "B.Cu") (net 3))
 (segment (start 216.071 120.611) (end 218.5 123.04) (width 0.2) (layer "B.Cu") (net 3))
 (segment (start 182.11 111.7) (end 186.03 115.62) (width 0.2) (layer "F.Cu") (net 9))
 (segment (start 186.03 115.62) (end 211.5 115.62) (width 0.2) (layer "F.Cu") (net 9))
 (segment (start 188.649 108.079) (end 209.71324 108.079) (width 0.2) (layer "F.Cu") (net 10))
 (segment (start 212.651 110.06324) (end 212.651 111.929) (width 0.2) (layer "F.Cu") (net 10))
 (segment (start 211.02324 109.389) (end 211.97676 109.389) (width 0.2) (layer "F.Cu") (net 10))
 (segment (start 209.71324 108.079) (end 211.02324 109.389) (width 0.2) (layer "F.Cu") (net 10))
 (segment (start 182.11 101.54) (end 188.649 108.079) (width 0.2) (layer "F.Cu") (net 10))
 (segment (start 211.97676 109.389) (end 212.651 110.06324) (width 0.2) (layer "F.Cu") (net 10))
 (segment (start 212.651 111.929) (end 211.5 113.08) (width 0.2) (layer "F.Cu") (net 10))
 (segment (start 182.11 106.62) (end 186.03 110.54) (width 0.2) (layer "F.Cu") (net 11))
 (segment (start 186.03 110.54) (end 211.5 110.54) (width 0.2) (layer "F.Cu") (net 11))
 (segment (start 207.361 125.481) (end 211.5 129.62) (width 0.2) (layer "F.Cu") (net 5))
 (segment (start 193.351 125.481) (end 207.361 125.481) (width 0.2) (layer "F.Cu") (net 5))
 (segment (start 182.11 114.24) (end 193.351 125.481) (width 0.2) (layer "F.Cu") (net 5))
 (segment (start 182.557765 112.781) (end 193.095765 123.319) (width 0.2) (layer "F.Cu") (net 6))
 (segment (start 181.662235 112.781) (end 182.557765 112.781) (width 0.2) (layer "F.Cu") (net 6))
 (segment (start 207.739 123.319) (end 211.5 127.08) (width 0.2) (layer "F.Cu") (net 6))
 (segment (start 182.11 104.08) (end 181.029 105.161) (width 0.2) (layer "F.Cu") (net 6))
 (segment (start 181.029 112.147765) (end 181.662235 112.781) (width 0.2) (layer "F.Cu") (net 6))
 (segment (start 181.029 105.161) (end 181.029 112.147765) (width 0.2) (layer "F.Cu") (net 6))
 (segment (start 193.095765 123.319) (end 207.739 123.319) (width 0.2) (layer "F.Cu") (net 6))
 (segment (start 212.651 116.771) (end 211.729 116.771) (width 0.2) (layer "F.Cu") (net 7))
 (segment (start 212.651 114.469) (end 212.651 116.771) (width 0.2) (layer "F.Cu") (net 7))
 (segment (start 210.349 114.469) (end 212.651 114.469) (width 0.2) (layer "F.Cu") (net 7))
 (segment (start 210.349 118.151) (end 210.349 123.389) (width 0.2) (layer "F.Cu") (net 7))
 (segment (start 186.109 113.159) (end 209.039 113.159) (width 0.2) (layer "F.Cu") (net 7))
 (segment (start 211.729 116.771) (end 210.349 118.151) (width 0.2) (layer "F.Cu") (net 7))
 (segment (start 182.11 109.16) (end 186.109 113.159) (width 0.2) (layer "F.Cu") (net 7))
 (segment (start 210.349 123.389) (end 211.5 124.54) (width 0.2) (layer "F.Cu") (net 7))
 (segment (start 209.039 113.159) (end 210.349 114.469) (width 0.2) (layer "F.Cu") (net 7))
 (segment (start 215.5 107) (end 218.5 110) (width 0.2) (layer "F.Cu") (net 12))
 (segment (start 206.93 106) (end 208 106) (width 0.2) (layer "F.Cu") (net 12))
 (segment (start 205.01 104.08) (end 206.93 106) (width 0.2) (layer "F.Cu") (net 12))
 (segment (start 215 107) (end 215.5 107) (width 0.2) (layer "F.Cu") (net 12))
 (via (at 208 106) (size 0.6) (drill 0.3) (layers "F.Cu" "B.Cu") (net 12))
 (via (at 215 107) (size 0.6) (drill 0.3) (layers "F.Cu" "B.Cu") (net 12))
 (segment (start 214.611 106.611) (end 215 107) (width 0.2) (layer "B.Cu") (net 12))
 (segment (start 208 106) (end 208.611 106.611) (width 0.2) (layer "B.Cu") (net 12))
 (segment (start 208.611 106.611) (end 214.611 106.611) (width 0.2) (layer "B.Cu") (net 12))
 (segment (start 205.71424 101.54) (end 211.02324 106.849) (width 0.2) (layer "F.Cu") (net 13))
 (segment (start 211.02324 106.849) (end 212.809 106.849) (width 0.2) (layer "F.Cu") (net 13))
 (segment (start 205.01 101.54) (end 205.71424 101.54) (width 0.2) (layer "F.Cu") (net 13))
 (segment (start 212.809 106.849) (end 218.5 112.54) (width 0.2) (layer "F.Cu") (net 13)))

